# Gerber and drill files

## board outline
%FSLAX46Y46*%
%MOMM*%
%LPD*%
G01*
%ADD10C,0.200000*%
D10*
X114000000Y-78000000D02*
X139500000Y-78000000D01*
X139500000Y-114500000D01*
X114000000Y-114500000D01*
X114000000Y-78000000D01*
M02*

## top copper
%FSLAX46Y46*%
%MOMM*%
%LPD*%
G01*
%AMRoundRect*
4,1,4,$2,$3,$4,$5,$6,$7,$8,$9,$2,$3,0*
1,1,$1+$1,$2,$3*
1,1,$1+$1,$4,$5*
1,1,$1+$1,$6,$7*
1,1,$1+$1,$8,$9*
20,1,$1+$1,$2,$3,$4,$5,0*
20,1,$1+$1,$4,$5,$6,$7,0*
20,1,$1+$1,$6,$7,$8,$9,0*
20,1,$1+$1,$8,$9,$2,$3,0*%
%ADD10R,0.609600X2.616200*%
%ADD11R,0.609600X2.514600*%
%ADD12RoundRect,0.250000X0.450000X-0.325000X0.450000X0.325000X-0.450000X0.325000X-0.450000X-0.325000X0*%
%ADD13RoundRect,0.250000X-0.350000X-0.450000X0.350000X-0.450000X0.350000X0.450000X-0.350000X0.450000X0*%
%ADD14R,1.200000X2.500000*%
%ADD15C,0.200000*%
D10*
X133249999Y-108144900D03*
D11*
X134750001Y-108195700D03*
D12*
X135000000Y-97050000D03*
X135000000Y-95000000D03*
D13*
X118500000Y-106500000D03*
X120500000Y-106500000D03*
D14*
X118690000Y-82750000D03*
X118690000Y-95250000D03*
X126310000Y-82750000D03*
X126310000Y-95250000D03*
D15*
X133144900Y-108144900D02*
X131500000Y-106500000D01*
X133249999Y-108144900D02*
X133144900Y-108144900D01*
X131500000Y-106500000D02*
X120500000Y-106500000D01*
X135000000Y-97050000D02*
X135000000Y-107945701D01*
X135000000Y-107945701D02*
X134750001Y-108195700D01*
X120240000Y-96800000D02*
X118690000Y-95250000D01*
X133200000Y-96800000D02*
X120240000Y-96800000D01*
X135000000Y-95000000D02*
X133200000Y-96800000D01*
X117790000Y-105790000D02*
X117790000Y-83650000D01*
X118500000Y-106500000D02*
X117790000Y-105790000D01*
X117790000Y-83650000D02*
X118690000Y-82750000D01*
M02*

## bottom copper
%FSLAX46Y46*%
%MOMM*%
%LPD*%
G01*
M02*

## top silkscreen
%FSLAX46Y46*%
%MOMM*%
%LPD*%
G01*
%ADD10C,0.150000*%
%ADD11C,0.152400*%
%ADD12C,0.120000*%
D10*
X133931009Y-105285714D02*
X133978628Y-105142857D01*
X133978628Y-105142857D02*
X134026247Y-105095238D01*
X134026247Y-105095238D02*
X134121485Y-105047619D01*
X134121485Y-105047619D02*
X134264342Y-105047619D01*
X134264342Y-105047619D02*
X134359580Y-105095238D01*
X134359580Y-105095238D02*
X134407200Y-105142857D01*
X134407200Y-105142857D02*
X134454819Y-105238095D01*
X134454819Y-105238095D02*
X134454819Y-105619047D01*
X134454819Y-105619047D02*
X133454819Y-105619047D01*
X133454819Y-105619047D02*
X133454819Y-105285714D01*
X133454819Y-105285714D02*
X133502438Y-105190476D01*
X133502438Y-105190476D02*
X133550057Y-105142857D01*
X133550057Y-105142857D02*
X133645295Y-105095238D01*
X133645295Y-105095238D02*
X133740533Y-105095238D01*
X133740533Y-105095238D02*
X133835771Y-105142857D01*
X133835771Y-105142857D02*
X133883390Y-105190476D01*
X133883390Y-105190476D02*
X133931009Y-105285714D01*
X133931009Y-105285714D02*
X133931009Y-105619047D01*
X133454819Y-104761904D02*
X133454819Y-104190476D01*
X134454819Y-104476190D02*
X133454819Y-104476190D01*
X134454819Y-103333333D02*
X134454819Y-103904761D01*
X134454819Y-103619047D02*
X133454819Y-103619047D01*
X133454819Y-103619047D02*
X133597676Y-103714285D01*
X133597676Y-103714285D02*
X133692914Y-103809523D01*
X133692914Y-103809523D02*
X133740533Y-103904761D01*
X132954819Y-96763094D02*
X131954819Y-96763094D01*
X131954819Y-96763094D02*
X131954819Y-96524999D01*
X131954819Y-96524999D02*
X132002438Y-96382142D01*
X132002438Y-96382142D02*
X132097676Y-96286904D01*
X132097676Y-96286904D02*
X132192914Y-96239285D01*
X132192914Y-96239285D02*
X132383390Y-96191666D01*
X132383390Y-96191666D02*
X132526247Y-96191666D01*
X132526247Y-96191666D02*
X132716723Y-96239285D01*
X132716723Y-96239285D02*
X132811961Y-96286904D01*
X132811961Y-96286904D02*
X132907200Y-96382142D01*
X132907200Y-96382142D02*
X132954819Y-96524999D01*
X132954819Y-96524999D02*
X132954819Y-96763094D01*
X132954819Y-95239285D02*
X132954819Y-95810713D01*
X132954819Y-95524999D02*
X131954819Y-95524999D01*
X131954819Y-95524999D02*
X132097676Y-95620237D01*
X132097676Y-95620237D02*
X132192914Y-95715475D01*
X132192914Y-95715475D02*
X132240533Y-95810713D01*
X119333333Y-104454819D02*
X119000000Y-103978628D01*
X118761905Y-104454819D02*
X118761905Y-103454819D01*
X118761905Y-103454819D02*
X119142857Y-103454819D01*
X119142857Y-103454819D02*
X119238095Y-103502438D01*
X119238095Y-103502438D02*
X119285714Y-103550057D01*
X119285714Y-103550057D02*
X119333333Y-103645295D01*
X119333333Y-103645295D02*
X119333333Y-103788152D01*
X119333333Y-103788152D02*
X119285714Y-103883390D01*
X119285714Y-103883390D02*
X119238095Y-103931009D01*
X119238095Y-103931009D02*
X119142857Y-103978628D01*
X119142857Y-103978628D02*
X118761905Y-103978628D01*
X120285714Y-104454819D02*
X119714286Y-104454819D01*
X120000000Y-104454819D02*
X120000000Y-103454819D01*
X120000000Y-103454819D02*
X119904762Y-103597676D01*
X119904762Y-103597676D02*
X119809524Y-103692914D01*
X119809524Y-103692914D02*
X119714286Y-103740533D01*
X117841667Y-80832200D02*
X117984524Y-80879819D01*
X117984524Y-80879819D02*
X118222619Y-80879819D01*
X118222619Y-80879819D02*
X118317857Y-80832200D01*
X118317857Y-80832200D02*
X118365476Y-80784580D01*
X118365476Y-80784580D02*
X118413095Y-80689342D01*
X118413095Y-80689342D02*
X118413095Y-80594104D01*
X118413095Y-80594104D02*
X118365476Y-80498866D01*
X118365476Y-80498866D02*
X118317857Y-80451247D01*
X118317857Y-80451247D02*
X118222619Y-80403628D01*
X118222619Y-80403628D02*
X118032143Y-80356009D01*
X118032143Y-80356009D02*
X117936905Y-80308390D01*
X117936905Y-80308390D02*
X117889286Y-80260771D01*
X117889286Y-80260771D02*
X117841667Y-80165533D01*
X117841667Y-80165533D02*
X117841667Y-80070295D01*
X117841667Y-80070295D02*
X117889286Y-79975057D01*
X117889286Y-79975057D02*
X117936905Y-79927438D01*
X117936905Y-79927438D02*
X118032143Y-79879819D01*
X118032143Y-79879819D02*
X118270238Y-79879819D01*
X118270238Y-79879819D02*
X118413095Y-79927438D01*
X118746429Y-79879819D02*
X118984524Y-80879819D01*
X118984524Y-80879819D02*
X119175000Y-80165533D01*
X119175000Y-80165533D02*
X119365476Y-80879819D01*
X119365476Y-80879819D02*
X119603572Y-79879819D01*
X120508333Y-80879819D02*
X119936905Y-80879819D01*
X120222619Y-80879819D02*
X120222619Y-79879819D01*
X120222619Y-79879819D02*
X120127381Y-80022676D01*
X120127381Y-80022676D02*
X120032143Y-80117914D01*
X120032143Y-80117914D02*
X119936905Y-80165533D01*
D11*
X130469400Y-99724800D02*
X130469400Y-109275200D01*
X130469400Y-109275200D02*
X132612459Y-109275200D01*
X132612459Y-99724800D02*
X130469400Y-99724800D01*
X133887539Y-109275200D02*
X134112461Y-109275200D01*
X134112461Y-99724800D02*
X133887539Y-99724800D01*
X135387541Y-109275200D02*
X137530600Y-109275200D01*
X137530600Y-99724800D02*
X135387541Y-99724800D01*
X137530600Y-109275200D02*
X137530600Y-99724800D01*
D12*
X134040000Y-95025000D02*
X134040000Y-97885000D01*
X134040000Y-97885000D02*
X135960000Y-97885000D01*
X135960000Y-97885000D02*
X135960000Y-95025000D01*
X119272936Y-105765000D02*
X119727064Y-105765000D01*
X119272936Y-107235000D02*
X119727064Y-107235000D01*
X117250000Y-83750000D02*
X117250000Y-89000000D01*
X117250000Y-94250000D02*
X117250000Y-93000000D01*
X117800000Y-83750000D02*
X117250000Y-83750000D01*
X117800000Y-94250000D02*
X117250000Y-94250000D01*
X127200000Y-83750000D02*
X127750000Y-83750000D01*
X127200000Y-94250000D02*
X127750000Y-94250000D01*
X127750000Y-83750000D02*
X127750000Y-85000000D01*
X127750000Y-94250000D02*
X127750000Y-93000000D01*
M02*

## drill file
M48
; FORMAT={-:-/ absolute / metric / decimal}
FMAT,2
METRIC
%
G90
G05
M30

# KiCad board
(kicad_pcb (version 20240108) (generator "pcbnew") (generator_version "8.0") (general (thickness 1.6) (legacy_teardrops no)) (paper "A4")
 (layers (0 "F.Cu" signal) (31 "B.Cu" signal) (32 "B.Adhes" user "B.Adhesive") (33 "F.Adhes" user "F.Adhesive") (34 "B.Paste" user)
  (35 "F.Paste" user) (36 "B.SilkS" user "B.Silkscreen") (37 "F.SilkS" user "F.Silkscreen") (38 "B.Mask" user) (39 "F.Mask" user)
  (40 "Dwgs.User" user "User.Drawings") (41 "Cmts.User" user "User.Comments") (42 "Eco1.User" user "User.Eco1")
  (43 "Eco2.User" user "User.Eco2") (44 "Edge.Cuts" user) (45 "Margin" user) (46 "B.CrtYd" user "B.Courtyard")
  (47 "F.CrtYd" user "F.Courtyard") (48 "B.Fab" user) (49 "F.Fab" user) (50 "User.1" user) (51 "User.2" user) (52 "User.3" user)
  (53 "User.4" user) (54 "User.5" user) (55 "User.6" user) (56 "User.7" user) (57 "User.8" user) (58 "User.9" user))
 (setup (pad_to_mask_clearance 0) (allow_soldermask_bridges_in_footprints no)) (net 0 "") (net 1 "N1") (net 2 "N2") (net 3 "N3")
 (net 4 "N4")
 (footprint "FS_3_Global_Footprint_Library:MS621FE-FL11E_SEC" (layer "F.Cu") (at 134 104.5 90)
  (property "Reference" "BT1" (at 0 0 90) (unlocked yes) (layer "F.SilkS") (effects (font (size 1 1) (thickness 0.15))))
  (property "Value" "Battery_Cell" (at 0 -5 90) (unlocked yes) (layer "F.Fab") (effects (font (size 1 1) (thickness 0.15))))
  (fp_line (start 4.7752 -3.5306) (end -4.7752 -3.5306) (stroke (width 0.1524) (type solid)) (layer "F.SilkS"))
  (fp_line (start -4.7752 -3.5306) (end -4.7752 -1.387541) (stroke (width 0.1524) (type solid)) (layer "F.SilkS"))
  (fp_line (start 4.7752 -1.387541) (end 4.7752 -3.5306) (stroke (width 0.1524) (type solid)) (layer "F.SilkS"))
  (fp_line (start -4.7752 -0.112461) (end -4.7752 0.112461) (stroke (width 0.1524) (type solid)) (layer "F.SilkS"))
  (fp_line (start 4.7752 0.112461) (end 4.7752 -0.112461) (stroke (width 0.1524) (type solid)) (layer "F.SilkS"))
  (fp_line (start -4.7752 1.387541) (end -4.7752 3.5306) (stroke (width 0.1524) (type solid)) (layer "F.SilkS"))
  (fp_line (start 4.7752 3.5306) (end 4.7752 1.387541) (stroke (width 0.1524) (type solid)) (layer "F.SilkS"))
  (fp_line (start -4.7752 3.5306) (end 4.7752 3.5306) (stroke (width 0.1524) (type solid)) (layer "F.SilkS"))
  (pad "1" smd rect (at -3.6449 -0.750001 90) (size 2.6162 0.6096) (layers "F.Cu" "F.Paste" "F.Mask") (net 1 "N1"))
  (pad "2" smd rect (at -3.6957 0.750001 90) (size 2.5146 0.6096) (layers "F.Cu" "F.Paste" "F.Mask") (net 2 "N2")))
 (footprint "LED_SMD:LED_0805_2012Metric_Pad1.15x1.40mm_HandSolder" (layer "F.Cu") (at 135 96.025 90)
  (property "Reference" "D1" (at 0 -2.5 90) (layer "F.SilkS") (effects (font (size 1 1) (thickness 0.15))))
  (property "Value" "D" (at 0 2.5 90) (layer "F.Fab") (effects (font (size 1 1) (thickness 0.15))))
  (fp_line (start 1 -0.96) (end -1.86 -0.96) (stroke (width 0.12) (type solid)) (layer "F.SilkS"))
  (fp_line (start -1.86 -0.96) (end -1.86 0.96) (stroke (width 0.12) (type solid)) (layer "F.SilkS"))
  (fp_line (start -1.86 0.96) (end 1 0.96) (stroke (width 0.12) (type solid)) (layer "F.SilkS"))
  (pad "1" smd roundrect (at -1.025 0 90) (size 1.15 1.4) (layers "F.Cu" "F.Paste" "F.Mask") (roundrect_rratio 0.217391) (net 2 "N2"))
  (pad "2" smd roundrect (at 1.025 0 90) (size 1.15 1.4) (layers "F.Cu" "F.Paste" "F.Mask") (roundrect_rratio 0.217391) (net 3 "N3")))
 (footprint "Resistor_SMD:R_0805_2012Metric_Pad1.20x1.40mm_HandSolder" (layer "F.Cu") (at 119.5 106.5)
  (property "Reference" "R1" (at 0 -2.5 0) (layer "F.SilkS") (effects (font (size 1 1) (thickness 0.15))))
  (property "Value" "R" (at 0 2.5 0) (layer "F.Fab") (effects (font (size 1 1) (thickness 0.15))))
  (fp_line (start -0.227064 -0.735) (end 0.227064 -0.735) (stroke (width 0.12) (type solid)) (layer "F.SilkS"))
  (fp_line (start -0.227064 0.735) (end 0.227064 0.735) (stroke (width 0.12) (type solid)) (layer "F.SilkS"))
  (pad "1" smd roundrect (at -1 0) (size 1.2 1.4) (layers "F.Cu" "F.Paste" "F.Mask") (roundrect_rratio 0.208333) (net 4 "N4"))
  (pad "2" smd roundrect (at 1 0) (size 1.2 1.4) (layers "F.Cu" "F.Paste" "F.Mask") (roundrect_rratio 0.208333) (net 1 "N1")))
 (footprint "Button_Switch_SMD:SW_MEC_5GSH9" (layer "F.Cu") (at 122.5 89)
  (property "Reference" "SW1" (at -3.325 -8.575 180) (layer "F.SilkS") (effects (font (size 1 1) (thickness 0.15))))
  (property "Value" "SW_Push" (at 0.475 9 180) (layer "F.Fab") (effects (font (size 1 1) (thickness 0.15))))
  (fp_line (start -5.25 -5.25) (end -5.25 0) (stroke (width 0.12) (type solid)) (layer "F.SilkS"))
  (fp_line (start -5.25 5.25) (end -5.25 4) (stroke (width 0.12) (type solid)) (layer "F.SilkS"))
  (fp_line (start -4.7 -5.25) (end -5.25 -5.25) (stroke (width 0.12) (type solid)) (layer "F.SilkS"))
  (fp_line (start -4.7 5.25) (end -5.25 5.25) (stroke (width 0.12) (type solid)) (layer "F.SilkS"))
  (fp_line (start 4.7 -5.25) (end 5.25 -5.25) (stroke (width 0.12) (type solid)) (layer "F.SilkS"))
  (fp_line (start 4.7 5.25) (end 5.25 5.25) (stroke (width 0.12) (type solid)) (layer "F.SilkS"))
  (fp_line (start 5.25 -5.25) (end 5.25 -4) (stroke (width 0.12) (type solid)) (layer "F.SilkS"))
  (fp_line (start 5.25 5.25) (end 5.25 4) (stroke (width 0.12) (type solid)) (layer "F.SilkS"))
  (pad "1" smd rect (at -3.81 -6.25 90) (size 2.5 1.2) (layers "F.Cu" "F.Paste" "F.Mask") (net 4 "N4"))
  (pad "2" smd rect (at -3.81 6.25 90) (size 2.5 1.2) (layers "F.Cu" "F.Paste" "F.Mask") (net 3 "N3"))
  (pad "3" smd rect (at 3.81 -6.25 90) (size 2.5 1.2) (layers "F.Cu" "F.Paste" "F.Mask"))
  (pad "4" smd rect (at 3.81 6.25 90) (size 2.5 1.2) (layers "F.Cu" "F.Paste" "F.Mask")))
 (gr_rect (start 114 78) (end 139.5 114.5) (stroke (width 0.2) (type default)) (fill none) (layer "Edge.Cuts"))
 (segment (start 133.1449 108.1449) (end 131.5 106.5) (width 0.2) (layer "F.Cu") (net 1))
 (segment (start 133.249999 108.1449) (end 133.1449 108.1449) (width 0.2) (layer "F.Cu") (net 1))
 (segment (start 131.5 106.5) (end 120.5 106.5) (width 0.2) (layer "F.Cu") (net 1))
 (segment (start 135 97.05) (end 135 107.945701) (width 0.2) (layer "F.Cu") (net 2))
 (segment (start 135 107.945701) (end 134.750001 108.1957) (width 0.2) (layer "F.Cu") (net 2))
 (segment (start 120.24 96.8) (end 118.69 95.25) (width 0.2) (layer "F.Cu") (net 3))
 (segment (start 133.2 96.8) (end 120.24 96.8) (width 0.2) (layer "F.Cu") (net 3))
 (segment (start 135 95) (end 133.2 96.8) (width 0.2) (layer "F.Cu") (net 3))
 (segment (start 117.79 105.79) (end 117.79 83.65) (width 0.2) (layer "F.Cu") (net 4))
 (segment (start 118.5 106.5) (end 117.79 105.79) (width 0.2) (layer "F.Cu") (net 4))
 (segment (start 117.79 83.65) (end 118.69 82.75) (width 0.2) (layer "F.Cu") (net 4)))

